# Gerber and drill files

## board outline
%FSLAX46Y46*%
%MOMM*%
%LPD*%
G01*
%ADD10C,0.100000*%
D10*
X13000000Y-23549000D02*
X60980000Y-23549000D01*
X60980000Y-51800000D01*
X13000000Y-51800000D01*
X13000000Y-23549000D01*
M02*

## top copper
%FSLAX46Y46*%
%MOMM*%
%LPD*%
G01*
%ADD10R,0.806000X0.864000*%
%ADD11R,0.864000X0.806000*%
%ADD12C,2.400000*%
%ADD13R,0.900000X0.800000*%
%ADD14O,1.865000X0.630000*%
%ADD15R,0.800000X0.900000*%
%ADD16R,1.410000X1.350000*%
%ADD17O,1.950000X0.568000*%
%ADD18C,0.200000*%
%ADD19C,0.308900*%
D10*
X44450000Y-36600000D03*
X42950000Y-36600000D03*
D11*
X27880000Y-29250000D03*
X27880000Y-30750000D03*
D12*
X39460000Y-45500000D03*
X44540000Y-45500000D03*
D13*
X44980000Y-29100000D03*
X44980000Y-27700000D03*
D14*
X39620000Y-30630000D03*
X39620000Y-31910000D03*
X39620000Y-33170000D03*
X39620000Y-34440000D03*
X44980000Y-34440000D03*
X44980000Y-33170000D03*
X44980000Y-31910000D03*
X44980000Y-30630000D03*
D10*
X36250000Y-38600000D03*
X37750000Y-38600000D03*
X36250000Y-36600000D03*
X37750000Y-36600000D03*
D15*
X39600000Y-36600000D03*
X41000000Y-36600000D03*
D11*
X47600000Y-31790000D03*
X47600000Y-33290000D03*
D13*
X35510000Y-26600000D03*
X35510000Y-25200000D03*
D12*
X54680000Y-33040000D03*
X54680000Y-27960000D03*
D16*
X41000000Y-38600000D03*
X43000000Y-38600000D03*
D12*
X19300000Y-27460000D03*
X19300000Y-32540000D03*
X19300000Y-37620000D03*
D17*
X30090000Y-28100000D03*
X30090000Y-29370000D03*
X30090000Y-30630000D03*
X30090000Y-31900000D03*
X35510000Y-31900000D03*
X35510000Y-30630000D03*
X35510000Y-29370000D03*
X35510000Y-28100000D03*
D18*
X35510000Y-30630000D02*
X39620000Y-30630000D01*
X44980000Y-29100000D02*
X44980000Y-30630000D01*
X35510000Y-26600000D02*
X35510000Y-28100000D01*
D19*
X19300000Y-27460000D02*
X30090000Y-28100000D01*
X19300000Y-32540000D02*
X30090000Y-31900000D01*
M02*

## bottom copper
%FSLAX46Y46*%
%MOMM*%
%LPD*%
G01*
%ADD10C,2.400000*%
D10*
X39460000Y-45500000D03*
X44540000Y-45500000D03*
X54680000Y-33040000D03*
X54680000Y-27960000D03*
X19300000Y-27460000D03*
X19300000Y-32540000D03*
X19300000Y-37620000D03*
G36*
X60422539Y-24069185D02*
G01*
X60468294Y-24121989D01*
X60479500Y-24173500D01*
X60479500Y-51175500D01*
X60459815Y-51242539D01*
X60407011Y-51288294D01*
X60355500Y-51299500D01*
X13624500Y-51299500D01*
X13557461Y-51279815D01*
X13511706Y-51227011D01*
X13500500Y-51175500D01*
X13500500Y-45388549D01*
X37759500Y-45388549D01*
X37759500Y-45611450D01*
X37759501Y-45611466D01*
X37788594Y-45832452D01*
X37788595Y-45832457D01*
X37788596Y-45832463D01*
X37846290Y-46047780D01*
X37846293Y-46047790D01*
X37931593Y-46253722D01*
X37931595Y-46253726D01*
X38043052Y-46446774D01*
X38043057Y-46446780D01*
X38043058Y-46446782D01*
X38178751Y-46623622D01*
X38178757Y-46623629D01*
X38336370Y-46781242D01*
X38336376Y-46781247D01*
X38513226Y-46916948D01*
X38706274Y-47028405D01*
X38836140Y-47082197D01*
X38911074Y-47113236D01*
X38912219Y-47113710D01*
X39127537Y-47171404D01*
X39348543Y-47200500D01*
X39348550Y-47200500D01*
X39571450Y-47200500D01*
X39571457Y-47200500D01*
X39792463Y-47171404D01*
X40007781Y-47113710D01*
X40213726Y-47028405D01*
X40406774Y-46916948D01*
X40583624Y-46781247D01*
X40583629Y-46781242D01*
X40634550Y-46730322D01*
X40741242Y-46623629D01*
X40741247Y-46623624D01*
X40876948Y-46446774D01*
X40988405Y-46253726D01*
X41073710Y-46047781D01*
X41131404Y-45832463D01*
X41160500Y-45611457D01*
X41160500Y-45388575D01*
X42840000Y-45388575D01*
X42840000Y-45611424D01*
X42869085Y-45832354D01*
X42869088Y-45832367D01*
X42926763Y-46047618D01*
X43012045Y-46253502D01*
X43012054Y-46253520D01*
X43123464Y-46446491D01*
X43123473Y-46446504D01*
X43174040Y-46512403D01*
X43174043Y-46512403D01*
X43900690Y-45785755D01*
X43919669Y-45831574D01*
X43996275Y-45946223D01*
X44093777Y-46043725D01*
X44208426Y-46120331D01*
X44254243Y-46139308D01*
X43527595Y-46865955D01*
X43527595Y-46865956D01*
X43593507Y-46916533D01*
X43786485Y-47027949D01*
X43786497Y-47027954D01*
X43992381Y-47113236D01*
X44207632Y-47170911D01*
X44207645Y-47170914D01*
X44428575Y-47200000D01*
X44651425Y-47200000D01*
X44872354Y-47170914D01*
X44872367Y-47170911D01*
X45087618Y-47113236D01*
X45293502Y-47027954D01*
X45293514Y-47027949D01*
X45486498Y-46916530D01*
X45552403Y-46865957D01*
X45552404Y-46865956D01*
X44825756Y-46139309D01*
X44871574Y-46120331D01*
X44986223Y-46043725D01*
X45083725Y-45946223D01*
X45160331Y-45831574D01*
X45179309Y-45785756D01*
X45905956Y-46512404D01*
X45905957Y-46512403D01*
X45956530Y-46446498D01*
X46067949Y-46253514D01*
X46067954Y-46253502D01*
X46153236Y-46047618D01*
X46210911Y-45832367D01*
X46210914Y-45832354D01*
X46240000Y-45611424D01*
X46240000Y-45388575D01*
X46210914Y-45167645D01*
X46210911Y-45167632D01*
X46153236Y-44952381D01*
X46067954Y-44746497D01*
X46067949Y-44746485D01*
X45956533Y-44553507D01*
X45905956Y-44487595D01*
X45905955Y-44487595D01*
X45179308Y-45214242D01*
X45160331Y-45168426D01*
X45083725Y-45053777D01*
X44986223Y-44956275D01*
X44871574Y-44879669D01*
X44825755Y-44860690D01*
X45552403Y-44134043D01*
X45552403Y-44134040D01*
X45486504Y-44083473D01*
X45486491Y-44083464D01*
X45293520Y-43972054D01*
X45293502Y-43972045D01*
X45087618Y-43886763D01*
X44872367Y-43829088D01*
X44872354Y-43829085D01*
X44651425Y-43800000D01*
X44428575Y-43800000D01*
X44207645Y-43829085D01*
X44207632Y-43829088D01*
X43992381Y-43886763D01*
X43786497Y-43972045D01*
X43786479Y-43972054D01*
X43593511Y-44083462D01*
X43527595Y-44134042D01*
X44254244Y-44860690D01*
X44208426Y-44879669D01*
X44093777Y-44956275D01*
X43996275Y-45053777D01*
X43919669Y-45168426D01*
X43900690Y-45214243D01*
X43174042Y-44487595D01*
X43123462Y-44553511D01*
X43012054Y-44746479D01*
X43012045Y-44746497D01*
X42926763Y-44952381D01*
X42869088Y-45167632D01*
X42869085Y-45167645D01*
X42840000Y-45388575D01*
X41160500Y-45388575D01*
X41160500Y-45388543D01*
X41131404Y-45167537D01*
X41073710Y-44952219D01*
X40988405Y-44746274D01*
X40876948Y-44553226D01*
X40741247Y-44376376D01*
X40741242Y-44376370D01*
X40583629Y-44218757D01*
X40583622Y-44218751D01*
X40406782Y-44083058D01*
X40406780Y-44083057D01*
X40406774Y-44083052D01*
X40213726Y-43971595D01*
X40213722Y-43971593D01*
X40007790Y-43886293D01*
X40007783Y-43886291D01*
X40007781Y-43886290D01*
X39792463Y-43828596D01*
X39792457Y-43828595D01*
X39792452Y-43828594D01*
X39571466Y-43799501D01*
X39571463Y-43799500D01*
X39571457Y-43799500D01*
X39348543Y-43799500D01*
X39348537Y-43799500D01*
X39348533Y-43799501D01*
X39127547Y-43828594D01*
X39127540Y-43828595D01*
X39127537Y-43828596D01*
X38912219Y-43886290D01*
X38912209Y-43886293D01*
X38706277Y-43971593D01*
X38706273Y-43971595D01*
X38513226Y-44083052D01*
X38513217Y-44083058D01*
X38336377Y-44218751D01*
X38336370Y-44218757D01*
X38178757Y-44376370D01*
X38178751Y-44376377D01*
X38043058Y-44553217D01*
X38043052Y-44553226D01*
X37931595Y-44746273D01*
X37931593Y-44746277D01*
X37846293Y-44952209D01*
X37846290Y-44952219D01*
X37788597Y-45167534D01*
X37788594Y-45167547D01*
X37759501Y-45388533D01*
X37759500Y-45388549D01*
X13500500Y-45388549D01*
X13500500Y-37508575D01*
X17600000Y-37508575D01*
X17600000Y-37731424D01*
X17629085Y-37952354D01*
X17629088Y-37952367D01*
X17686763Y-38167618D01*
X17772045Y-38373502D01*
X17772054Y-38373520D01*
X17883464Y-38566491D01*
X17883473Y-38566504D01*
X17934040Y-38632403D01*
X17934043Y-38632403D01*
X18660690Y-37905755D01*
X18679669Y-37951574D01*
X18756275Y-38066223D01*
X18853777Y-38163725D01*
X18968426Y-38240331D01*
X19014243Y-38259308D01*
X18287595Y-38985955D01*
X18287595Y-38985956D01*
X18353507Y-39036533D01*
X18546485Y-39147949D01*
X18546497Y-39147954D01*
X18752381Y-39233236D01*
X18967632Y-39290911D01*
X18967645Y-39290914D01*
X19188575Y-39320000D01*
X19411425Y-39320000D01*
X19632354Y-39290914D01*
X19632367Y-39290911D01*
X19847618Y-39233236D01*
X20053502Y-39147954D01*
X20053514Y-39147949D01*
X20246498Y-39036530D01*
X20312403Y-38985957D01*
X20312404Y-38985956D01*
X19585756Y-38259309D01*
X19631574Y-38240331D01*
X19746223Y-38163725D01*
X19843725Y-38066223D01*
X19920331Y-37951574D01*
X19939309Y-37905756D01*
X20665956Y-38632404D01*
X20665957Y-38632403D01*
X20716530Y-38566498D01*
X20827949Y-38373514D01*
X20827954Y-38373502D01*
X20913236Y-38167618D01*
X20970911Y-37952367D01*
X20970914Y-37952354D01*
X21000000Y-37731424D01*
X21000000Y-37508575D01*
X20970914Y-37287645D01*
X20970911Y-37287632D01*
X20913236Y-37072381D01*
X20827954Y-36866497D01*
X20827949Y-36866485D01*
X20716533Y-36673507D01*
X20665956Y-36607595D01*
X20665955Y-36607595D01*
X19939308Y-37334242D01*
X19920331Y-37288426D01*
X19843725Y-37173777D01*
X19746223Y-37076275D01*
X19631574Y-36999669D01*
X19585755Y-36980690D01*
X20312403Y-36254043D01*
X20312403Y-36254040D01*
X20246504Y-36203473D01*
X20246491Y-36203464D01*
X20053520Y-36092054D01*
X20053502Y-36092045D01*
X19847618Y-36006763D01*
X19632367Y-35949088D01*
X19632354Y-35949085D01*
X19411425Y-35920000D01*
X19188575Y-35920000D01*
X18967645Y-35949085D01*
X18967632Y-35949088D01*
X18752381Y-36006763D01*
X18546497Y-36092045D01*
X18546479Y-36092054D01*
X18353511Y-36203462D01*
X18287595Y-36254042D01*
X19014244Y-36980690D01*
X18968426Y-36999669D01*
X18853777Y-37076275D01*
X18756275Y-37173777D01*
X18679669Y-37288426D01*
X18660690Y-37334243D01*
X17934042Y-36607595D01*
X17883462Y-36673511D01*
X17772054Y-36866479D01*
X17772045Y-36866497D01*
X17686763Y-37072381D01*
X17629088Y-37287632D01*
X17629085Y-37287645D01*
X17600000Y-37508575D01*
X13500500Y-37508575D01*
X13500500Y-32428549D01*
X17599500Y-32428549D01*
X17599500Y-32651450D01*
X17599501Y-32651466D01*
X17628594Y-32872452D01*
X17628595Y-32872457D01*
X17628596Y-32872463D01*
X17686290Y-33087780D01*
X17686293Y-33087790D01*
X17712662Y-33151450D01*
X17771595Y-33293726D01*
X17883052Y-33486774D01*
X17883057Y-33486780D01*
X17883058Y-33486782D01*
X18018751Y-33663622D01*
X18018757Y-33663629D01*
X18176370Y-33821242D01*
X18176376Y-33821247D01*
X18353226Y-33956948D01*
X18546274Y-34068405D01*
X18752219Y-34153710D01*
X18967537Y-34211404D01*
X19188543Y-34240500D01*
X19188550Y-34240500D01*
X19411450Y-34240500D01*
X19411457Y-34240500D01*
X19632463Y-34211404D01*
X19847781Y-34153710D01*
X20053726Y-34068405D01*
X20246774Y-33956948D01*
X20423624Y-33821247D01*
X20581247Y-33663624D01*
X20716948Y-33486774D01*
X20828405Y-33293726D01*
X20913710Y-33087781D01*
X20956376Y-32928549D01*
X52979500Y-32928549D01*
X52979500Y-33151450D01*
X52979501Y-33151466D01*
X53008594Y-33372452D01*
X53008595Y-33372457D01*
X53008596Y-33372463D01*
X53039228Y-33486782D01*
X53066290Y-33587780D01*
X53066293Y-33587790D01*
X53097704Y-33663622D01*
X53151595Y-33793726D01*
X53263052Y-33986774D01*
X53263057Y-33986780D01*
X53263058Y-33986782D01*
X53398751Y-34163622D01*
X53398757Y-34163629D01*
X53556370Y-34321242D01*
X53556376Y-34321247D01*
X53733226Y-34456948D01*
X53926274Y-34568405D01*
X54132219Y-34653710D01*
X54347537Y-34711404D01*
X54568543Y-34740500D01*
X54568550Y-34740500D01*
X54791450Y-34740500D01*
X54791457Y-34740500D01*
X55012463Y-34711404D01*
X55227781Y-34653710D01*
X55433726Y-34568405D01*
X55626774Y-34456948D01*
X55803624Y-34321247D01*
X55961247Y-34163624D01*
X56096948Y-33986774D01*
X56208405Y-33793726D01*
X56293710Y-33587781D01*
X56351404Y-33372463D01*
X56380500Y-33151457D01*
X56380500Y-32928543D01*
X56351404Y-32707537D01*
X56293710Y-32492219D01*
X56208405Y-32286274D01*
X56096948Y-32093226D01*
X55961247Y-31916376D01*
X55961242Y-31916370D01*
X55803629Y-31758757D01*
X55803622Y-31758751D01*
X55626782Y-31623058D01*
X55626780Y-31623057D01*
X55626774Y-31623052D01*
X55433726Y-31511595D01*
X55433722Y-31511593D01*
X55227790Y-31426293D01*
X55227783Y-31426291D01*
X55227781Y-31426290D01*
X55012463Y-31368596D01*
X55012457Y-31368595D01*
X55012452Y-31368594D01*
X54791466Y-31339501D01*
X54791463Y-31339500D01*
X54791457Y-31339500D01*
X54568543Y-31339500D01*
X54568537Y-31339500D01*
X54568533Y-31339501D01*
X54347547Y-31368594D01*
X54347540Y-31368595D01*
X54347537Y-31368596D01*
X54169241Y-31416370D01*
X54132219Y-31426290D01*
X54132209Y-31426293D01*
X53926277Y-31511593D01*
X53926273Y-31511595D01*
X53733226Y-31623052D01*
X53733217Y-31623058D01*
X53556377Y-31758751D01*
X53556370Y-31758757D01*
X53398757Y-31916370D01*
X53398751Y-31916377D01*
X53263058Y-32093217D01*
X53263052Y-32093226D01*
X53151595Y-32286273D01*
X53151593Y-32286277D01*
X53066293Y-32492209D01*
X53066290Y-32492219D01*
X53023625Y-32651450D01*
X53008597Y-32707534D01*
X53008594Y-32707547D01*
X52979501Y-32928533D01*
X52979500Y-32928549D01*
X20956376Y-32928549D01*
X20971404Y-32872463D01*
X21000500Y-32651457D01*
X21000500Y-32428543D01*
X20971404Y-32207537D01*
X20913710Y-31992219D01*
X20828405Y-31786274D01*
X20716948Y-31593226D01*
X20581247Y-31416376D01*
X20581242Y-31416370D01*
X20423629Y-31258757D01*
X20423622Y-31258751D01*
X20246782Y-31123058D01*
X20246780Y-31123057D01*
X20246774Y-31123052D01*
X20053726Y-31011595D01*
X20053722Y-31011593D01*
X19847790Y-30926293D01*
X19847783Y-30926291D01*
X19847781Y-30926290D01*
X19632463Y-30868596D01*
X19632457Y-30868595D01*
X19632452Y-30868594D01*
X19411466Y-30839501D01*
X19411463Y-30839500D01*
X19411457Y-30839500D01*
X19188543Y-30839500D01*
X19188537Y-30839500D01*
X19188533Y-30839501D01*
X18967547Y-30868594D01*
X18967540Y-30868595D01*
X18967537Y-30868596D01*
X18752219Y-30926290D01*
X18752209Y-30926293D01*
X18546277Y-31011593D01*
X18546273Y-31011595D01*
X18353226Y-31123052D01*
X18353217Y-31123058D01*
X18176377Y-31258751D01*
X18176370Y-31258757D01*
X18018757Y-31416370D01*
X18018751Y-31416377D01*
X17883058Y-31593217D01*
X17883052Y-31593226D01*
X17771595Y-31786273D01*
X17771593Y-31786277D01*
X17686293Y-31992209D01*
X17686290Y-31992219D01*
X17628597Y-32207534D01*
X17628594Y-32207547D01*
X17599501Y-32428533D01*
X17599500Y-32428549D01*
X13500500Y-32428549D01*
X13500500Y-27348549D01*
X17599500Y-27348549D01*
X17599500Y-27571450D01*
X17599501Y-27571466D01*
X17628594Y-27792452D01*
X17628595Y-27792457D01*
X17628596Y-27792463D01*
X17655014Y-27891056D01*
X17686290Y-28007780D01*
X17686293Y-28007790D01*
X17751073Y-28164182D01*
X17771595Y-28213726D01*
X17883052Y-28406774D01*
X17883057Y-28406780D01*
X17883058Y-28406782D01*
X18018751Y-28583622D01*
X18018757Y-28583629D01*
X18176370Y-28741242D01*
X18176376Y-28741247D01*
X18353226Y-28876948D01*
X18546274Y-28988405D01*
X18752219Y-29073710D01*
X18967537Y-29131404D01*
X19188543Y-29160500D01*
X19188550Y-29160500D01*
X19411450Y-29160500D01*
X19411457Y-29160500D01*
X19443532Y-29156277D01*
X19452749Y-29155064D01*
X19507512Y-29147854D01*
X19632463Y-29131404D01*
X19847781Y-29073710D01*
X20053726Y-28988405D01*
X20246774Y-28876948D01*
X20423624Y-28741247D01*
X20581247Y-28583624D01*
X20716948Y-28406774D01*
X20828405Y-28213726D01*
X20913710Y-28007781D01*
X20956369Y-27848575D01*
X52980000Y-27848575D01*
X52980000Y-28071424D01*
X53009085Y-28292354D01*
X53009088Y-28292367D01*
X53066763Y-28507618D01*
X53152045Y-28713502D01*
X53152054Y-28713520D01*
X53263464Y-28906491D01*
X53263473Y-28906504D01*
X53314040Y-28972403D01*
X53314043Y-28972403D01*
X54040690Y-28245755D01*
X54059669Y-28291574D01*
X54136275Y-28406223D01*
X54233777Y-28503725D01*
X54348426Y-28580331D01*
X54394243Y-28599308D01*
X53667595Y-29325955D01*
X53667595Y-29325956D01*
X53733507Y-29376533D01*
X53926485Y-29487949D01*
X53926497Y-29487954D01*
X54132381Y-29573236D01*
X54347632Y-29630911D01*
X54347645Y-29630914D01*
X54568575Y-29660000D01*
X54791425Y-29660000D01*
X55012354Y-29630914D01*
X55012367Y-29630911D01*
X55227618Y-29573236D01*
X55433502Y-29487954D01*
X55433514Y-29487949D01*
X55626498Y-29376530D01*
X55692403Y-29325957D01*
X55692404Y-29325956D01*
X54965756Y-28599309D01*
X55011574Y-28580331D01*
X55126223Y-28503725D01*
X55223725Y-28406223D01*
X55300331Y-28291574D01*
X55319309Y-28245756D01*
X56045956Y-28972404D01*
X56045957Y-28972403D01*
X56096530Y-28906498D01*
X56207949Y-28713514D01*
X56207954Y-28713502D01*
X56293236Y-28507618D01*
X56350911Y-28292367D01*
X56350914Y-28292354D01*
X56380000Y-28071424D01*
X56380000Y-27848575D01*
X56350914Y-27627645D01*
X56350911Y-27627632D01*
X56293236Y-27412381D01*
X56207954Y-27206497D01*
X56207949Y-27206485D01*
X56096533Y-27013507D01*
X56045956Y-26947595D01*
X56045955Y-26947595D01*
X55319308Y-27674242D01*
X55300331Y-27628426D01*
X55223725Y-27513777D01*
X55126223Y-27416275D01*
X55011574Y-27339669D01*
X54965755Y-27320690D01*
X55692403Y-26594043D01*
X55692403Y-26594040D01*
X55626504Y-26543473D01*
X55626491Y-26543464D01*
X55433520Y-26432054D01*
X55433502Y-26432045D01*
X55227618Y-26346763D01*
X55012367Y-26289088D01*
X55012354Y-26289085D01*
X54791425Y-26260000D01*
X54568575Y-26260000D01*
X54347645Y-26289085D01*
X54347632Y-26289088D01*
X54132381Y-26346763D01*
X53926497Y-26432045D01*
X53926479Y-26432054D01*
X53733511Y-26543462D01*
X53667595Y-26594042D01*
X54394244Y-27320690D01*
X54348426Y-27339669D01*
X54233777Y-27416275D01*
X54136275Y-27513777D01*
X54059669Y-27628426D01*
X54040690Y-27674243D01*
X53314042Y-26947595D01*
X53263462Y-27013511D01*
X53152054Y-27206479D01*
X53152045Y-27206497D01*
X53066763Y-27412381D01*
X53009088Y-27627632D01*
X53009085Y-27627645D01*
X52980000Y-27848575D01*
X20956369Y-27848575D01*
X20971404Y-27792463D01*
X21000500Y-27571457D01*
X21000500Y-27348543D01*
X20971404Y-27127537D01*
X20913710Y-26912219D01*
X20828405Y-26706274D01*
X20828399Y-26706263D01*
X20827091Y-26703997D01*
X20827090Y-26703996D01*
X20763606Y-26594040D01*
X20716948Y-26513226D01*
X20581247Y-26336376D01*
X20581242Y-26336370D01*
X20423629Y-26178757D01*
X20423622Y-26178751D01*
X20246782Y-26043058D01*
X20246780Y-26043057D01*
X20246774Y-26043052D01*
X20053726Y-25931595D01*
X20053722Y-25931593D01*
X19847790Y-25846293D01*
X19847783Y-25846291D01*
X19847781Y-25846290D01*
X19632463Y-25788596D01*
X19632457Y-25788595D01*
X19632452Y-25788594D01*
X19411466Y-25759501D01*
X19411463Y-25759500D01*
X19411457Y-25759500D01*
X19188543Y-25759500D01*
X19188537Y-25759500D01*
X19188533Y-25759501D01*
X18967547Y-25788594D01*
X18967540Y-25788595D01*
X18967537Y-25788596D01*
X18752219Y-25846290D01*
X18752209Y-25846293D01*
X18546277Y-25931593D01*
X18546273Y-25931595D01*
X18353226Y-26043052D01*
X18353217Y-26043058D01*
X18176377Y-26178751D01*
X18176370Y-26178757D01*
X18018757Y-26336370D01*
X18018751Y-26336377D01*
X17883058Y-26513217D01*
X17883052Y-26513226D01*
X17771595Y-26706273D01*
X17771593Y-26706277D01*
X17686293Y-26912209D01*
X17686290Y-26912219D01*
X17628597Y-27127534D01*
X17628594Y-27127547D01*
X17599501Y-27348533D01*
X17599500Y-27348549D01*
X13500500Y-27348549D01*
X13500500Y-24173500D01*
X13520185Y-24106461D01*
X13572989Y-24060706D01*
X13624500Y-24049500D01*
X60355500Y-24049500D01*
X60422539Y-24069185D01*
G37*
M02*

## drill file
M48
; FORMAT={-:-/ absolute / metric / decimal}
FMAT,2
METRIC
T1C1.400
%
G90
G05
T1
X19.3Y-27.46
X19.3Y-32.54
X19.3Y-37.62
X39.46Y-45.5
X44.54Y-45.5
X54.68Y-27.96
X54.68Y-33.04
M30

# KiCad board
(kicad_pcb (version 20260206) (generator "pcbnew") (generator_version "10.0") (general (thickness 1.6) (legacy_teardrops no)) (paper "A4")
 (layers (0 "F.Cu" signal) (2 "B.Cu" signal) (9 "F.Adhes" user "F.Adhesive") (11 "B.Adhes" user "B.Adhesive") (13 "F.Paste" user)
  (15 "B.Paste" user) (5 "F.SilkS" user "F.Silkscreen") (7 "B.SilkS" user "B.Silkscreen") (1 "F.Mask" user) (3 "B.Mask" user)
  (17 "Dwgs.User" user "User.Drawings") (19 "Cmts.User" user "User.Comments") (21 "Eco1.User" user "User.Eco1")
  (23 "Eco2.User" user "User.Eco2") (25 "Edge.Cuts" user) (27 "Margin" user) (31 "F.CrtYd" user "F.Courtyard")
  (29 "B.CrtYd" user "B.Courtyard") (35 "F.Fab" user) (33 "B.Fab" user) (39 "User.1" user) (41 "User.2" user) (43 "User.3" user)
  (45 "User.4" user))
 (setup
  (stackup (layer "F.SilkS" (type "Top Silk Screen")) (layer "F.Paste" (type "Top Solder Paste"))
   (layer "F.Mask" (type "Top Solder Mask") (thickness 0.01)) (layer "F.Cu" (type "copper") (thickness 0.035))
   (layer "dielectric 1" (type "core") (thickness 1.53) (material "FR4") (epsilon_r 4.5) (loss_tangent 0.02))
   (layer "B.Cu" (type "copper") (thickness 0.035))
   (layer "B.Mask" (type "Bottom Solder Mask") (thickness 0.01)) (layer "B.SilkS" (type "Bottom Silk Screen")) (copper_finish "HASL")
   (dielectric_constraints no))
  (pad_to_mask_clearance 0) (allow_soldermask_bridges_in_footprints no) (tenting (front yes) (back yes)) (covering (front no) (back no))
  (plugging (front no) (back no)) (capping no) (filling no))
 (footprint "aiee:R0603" (layer "F.Cu") (at 43.7 36.6 180)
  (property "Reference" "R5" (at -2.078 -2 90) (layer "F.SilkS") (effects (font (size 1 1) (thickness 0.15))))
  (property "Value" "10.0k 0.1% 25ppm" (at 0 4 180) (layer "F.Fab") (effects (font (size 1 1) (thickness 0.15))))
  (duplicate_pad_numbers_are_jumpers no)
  (pad "1" smd rect (at -0.75 0 180) (size 0.806 0.864) (layers "F.Cu" "F.Mask" "F.Paste") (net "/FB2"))
  (pad "2" smd rect (at 0.75 0 180) (size 0.806 0.864) (layers "F.Cu" "F.Mask" "F.Paste") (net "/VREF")))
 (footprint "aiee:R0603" (layer "F.Cu") (at 27.88 30 -90)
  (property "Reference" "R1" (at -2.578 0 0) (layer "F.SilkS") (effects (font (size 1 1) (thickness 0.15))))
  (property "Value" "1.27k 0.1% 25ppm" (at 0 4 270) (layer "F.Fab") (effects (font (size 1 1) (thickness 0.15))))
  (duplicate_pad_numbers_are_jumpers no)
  (pad "1" smd rect (at -0.75 0 270) (size 0.806 0.864) (layers "F.Cu" "F.Mask" "F.Paste") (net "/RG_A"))
  (pad "2" smd rect (at 0.75 0 270) (size 0.806 0.864) (layers "F.Cu" "F.Mask" "F.Paste") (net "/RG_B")))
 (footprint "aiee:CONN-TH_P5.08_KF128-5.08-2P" (layer "F.Cu") (at 42 45.5)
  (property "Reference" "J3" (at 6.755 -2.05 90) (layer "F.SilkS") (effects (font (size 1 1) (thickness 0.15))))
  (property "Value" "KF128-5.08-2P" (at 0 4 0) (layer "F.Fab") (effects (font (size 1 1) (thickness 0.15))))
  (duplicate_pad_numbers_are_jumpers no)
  (pad "1" thru_hole circle (at -2.54 0) (size 2.4 2.4) (drill 1.399998) (layers "*.Cu" "*.Mask") (remove_unused_layers no) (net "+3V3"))
  (pad "2" thru_hole circle (at 2.54 0) (size 2.4 2.4) (drill 1.399998) (layers "*.Cu" "*.Mask") (remove_unused_layers no) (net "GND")))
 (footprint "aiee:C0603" (layer "F.Cu") (at 44.98 28.4 90)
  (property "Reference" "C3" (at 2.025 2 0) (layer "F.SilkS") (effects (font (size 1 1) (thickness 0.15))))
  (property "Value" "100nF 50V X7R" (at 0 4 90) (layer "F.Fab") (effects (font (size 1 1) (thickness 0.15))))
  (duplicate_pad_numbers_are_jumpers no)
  (pad "1" smd rect (at -0.7 0 90) (size 0.8 0.9) (layers "F.Cu" "F.Mask" "F.Paste") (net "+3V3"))
  (pad "2" smd rect (at 0.7 0 90) (size 0.8 0.9) (layers "F.Cu" "F.Mask" "F.Paste") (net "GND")))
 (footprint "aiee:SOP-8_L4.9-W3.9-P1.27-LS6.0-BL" (layer "F.Cu") (at 42.3 32.54 -90)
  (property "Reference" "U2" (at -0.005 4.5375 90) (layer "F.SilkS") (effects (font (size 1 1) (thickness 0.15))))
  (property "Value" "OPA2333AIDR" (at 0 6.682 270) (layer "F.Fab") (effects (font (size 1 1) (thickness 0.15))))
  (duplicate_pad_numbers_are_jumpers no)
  (pad "1" smd oval (at -1.91 2.68 270) (size 0.63 1.865) (layers "F.Cu" "F.Mask" "F.Paste") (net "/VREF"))
  (pad "2" smd oval (at -0.63 2.68 270) (size 0.63 1.865) (layers "F.Cu" "F.Mask" "F.Paste") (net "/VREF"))
  (pad "3" smd oval (at 0.63 2.68 270) (size 0.63 1.865) (layers "F.Cu" "F.Mask" "F.Paste") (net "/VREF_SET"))
  (pad "4" smd oval (at 1.9 2.68 270) (size 0.63 1.865) (layers "F.Cu" "F.Mask" "F.Paste") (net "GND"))
  (pad "5" smd oval (at 1.9 -2.68 270) (size 0.63 1.865) (layers "F.Cu" "F.Mask" "F.Paste") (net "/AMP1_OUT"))
  (pad "6" smd oval (at 0.63 -2.68 270) (size 0.63 1.865) (layers "F.Cu" "F.Mask" "F.Paste") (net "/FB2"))
  (pad "7" smd oval (at -0.63 -2.68 270) (size 0.63 1.865) (layers "F.Cu" "F.Mask" "F.Paste") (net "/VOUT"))
  (pad "8" smd oval (at -1.91 -2.68 270) (size 0.63 1.865) (layers "F.Cu" "F.Mask" "F.Paste") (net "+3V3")))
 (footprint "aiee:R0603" (layer "F.Cu") (at 37 38.6)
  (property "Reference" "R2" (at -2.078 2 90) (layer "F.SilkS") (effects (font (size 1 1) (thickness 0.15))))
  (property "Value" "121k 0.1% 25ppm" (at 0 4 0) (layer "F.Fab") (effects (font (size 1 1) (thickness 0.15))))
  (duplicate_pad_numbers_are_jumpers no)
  (pad "1" smd rect (at -0.75 0) (size 0.806 0.864) (layers "F.Cu" "F.Mask" "F.Paste") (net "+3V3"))
  (pad "2" smd rect (at 0.75 0) (size 0.806 0.864) (layers "F.Cu" "F.Mask" "F.Paste") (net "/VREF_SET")))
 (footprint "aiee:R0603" (layer "F.Cu") (at 37 36.6)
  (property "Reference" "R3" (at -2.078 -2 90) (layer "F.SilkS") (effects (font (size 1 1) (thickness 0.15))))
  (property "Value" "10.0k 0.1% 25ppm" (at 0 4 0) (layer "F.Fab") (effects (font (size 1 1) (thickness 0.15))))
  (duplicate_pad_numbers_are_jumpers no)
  (pad "1" smd rect (at -0.75 0) (size 0.806 0.864) (layers "F.Cu" "F.Mask" "F.Paste") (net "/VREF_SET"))
  (pad "2" smd rect (at 0.75 0) (size 0.806 0.864) (layers "F.Cu" "F.Mask" "F.Paste") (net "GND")))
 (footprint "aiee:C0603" (layer "F.Cu") (at 40.3 36.6)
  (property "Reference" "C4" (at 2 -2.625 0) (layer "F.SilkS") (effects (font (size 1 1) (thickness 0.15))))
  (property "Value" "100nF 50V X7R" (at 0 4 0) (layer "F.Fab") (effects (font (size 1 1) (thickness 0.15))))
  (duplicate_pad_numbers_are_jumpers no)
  (pad "1" smd rect (at -0.7 0) (size 0.8 0.9) (layers "F.Cu" "F.Mask" "F.Paste") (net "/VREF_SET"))
  (pad "2" smd rect (at 0.7 0) (size 0.8 0.9) (layers "F.Cu" "F.Mask" "F.Paste") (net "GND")))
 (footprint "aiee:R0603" (layer "F.Cu") (at 47.6 32.54 -90)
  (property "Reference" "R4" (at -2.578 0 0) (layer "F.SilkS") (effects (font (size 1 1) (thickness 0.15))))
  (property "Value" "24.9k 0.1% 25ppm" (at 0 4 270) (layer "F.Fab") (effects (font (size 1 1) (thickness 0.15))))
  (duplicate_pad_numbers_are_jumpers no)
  (pad "1" smd rect (at -0.75 0 270) (size 0.806 0.864) (layers "F.Cu" "F.Mask" "F.Paste") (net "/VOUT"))
  (pad "2" smd rect (at 0.75 0 270) (size 0.806 0.864) (layers "F.Cu" "F.Mask" "F.Paste") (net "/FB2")))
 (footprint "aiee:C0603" (layer "F.Cu") (at 35.51 25.9 90)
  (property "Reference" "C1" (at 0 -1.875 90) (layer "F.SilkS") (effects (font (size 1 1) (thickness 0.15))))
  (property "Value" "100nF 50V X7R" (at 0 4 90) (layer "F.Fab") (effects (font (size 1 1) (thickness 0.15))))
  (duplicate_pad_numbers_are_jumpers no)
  (pad "1" smd rect (at -0.7 0 90) (size 0.8 0.9) (layers "F.Cu" "F.Mask" "F.Paste") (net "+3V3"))
  (pad "2" smd rect (at 0.7 0 90) (size 0.8 0.9) (layers "F.Cu" "F.Mask" "F.Paste") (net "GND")))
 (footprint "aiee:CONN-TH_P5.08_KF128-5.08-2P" (layer "F.Cu") (at 54.68 30.5 90)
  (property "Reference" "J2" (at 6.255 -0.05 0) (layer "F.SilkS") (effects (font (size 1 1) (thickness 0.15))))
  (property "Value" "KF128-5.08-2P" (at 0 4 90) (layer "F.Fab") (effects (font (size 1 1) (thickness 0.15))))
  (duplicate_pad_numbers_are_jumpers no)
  (pad "1" thru_hole circle (at -2.54 0 90) (size 2.4 2.4) (drill 1.399998) (layers "*.Cu" "*.Mask") (remove_unused_layers no) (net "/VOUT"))
  (pad "2" thru_hole circle (at 2.54 0 90) (size 2.4 2.4) (drill 1.399998) (layers "*.Cu" "*.Mask") (remove_unused_layers no) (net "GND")))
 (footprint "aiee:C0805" (layer "F.Cu") (at 42 38.6)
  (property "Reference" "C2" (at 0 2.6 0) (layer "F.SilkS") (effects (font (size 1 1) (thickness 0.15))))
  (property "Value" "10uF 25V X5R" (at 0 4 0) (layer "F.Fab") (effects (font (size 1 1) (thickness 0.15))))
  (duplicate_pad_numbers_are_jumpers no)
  (pad "1" smd rect (at -1 0) (size 1.41 1.35) (layers "F.Cu" "F.Mask" "F.Paste") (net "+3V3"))
  (pad "2" smd rect (at 1 0) (size 1.41 1.35) (layers "F.Cu" "F.Mask" "F.Paste") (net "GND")))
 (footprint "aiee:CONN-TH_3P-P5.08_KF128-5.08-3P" (layer "F.Cu") (at 19.3 32.54 -90)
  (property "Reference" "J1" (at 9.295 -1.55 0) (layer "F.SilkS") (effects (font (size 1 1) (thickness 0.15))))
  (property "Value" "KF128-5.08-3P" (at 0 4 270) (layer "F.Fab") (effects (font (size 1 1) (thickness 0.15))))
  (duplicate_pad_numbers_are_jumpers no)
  (pad "1" thru_hole circle (at -5.08 0 270) (size 2.4 2.4) (drill 1.399998) (layers "*.Cu" "*.Mask") (remove_unused_layers no)
   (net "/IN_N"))
  (pad "2" thru_hole circle (at 0 0 270) (size 2.4 2.4) (drill 1.399998) (layers "*.Cu" "*.Mask") (remove_unused_layers no) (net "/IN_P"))
  (pad "3" thru_hole circle (at 5.08 0 270) (size 2.4 2.4) (drill 1.399998) (layers "*.Cu" "*.Mask") (remove_unused_layers no) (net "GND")))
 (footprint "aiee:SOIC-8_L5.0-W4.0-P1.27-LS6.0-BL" (layer "F.Cu") (at 32.8 30 -90)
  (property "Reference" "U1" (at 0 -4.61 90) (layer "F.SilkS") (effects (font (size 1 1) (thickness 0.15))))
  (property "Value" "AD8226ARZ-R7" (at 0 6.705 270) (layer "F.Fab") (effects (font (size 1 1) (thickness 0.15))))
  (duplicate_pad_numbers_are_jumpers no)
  (pad "1" smd oval (at -1.9 2.71 270) (size 0.568 1.95) (layers "F.Cu" "F.Mask" "F.Paste") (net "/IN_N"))
  (pad "2" smd oval (at -0.63 2.71 270) (size 0.568 1.95) (layers "F.Cu" "F.Mask" "F.Paste") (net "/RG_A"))
  (pad "3" smd oval (at 0.63 2.71 270) (size 0.568 1.95) (layers "F.Cu" "F.Mask" "F.Paste") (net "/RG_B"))
  (pad "4" smd oval (at 1.9 2.71 270) (size 0.568 1.95) (layers "F.Cu" "F.Mask" "F.Paste") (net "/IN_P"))
  (pad "5" smd oval (at 1.9 -2.71 270) (size 0.568 1.95) (layers "F.Cu" "F.Mask" "F.Paste") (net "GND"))
  (pad "6" smd oval (at 0.63 -2.71 270) (size 0.568 1.95) (layers "F.Cu" "F.Mask" "F.Paste") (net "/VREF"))
  (pad "7" smd oval (at -0.63 -2.71 270) (size 0.568 1.95) (layers "F.Cu" "F.Mask" "F.Paste") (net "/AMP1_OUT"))
  (pad "8" smd oval (at -1.9 -2.71 270) (size 0.568 1.95) (layers "F.Cu" "F.Mask" "F.Paste") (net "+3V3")))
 (gr_rect (start 13 23.549) (end 60.98 51.8) (stroke (width 0.1) (type default)) (fill no) (layer "Edge.Cuts"))
 (segment (start 35.51 30.63) (end 39.62 30.63) (width 0.2) (layer "F.Cu") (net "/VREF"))
 (segment (start 44.98 29.1) (end 44.98 30.63) (width 0.2) (layer "F.Cu") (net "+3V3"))
 (segment (start 35.51 26.6) (end 35.51 28.1) (width 0.2) (layer "F.Cu") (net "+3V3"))
 (segment (start 19.3 27.46) (end 30.09 28.1) (width 0.3089) (layer "F.Cu") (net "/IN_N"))
 (segment (start 19.3 32.54) (end 30.09 31.9) (width 0.3089) (layer "F.Cu") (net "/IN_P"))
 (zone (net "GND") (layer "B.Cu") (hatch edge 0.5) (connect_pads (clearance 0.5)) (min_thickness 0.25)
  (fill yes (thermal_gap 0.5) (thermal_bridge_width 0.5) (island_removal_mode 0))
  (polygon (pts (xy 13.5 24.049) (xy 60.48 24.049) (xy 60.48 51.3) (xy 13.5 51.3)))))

